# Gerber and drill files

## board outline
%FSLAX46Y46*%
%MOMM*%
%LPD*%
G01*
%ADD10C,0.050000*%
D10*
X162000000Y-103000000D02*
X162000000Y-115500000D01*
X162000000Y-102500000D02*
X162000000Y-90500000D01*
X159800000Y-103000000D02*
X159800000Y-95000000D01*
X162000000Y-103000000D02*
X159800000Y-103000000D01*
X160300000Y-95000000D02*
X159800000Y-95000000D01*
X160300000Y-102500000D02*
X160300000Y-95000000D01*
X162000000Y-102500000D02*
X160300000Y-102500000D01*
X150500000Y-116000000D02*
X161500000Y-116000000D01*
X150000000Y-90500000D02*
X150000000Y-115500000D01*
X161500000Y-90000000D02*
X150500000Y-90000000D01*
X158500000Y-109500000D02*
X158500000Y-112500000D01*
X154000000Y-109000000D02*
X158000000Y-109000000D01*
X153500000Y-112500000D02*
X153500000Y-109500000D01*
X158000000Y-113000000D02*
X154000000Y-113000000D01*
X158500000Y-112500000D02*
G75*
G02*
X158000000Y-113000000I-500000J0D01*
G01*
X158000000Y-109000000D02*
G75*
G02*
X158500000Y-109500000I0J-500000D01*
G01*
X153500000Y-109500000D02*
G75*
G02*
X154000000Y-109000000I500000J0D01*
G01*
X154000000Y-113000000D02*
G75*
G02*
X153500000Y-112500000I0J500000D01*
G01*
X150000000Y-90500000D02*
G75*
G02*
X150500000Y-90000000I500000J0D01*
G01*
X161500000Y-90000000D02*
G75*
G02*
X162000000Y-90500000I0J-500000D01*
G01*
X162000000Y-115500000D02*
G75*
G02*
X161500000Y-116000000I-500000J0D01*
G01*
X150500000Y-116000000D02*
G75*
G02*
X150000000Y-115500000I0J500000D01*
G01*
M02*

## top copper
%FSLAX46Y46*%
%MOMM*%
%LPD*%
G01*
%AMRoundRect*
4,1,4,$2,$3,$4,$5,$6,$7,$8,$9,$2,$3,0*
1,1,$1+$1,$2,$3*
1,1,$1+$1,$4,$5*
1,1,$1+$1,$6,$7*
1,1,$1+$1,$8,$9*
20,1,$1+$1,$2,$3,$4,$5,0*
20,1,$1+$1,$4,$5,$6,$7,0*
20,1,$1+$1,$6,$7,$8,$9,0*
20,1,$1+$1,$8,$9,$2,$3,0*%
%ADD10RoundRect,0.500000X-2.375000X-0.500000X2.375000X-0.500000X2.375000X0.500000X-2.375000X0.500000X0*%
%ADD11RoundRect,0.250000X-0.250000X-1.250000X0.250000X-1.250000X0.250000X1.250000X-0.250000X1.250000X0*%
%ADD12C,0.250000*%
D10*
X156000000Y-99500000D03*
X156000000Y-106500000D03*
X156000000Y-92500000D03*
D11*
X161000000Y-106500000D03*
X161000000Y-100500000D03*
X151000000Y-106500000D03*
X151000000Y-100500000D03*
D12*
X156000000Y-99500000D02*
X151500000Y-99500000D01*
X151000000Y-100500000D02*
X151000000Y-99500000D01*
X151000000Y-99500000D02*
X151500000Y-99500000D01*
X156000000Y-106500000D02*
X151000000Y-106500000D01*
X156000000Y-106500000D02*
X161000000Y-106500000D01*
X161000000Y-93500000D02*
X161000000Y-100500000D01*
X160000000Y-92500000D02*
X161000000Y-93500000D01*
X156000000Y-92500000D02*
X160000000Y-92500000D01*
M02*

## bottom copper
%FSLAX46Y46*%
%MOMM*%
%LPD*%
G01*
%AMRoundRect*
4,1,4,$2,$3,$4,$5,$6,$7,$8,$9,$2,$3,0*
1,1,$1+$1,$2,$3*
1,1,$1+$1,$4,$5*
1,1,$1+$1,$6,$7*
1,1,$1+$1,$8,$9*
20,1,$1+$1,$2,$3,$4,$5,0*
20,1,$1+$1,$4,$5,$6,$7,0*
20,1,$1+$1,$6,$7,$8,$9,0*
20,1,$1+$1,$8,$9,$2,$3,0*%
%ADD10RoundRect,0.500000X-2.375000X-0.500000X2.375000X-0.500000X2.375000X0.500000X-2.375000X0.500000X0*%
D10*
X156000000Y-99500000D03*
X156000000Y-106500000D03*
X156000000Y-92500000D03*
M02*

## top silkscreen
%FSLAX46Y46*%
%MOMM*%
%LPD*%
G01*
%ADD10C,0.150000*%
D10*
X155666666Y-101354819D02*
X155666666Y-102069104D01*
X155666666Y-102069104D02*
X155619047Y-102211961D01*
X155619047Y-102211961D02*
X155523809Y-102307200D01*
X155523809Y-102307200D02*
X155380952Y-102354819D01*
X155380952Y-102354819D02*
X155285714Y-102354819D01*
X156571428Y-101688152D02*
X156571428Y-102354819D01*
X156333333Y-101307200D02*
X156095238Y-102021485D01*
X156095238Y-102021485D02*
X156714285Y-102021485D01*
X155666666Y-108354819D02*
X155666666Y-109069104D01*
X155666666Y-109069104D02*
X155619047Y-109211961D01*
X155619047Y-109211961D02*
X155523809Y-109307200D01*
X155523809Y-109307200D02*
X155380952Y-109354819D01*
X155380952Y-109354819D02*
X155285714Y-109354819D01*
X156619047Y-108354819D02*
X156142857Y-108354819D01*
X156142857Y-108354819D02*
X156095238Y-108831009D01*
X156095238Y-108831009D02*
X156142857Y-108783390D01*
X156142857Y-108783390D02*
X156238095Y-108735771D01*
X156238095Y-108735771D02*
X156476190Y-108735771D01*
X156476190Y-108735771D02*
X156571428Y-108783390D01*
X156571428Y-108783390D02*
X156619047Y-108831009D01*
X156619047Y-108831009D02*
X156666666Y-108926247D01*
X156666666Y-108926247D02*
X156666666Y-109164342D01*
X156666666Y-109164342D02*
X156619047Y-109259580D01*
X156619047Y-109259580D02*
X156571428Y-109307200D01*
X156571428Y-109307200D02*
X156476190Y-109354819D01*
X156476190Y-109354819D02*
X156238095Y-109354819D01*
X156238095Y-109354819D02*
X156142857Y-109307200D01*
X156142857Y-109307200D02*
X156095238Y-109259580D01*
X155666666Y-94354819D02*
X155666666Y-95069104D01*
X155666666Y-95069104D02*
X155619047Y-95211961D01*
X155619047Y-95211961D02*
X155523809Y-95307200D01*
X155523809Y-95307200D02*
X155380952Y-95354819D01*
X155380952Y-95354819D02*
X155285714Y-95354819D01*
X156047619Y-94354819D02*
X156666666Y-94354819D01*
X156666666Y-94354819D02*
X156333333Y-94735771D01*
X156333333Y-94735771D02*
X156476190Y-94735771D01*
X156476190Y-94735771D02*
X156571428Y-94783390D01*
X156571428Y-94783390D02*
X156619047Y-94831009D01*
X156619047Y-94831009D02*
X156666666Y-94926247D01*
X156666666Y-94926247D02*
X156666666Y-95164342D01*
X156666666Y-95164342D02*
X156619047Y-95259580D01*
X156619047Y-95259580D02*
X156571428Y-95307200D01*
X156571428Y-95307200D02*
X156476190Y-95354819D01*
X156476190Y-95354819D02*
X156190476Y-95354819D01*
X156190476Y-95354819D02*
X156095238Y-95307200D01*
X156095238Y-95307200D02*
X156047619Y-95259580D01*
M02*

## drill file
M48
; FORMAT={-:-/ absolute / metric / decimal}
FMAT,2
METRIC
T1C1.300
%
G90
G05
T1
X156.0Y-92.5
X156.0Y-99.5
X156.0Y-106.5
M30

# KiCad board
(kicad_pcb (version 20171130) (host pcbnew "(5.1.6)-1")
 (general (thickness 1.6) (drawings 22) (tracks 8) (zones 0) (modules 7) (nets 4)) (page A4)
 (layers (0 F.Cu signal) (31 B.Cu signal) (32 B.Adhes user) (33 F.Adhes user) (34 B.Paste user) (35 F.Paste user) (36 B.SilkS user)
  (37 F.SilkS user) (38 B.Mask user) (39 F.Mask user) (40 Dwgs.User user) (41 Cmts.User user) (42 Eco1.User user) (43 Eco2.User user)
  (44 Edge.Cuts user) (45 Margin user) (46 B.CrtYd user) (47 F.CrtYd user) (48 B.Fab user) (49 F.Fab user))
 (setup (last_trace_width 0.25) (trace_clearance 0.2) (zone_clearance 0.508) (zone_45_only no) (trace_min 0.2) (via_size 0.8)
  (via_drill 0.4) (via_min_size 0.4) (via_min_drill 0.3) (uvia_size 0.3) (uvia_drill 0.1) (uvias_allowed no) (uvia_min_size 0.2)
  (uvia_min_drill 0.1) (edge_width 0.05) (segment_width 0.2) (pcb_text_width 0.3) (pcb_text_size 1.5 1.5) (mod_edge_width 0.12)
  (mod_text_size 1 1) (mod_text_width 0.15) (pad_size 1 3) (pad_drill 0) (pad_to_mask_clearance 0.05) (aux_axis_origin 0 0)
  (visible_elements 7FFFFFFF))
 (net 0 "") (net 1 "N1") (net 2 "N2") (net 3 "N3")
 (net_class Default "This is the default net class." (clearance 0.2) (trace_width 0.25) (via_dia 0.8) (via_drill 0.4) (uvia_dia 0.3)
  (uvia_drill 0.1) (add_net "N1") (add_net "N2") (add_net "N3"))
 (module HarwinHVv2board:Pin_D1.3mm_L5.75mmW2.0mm (layer F.Cu) (at 156 99.5)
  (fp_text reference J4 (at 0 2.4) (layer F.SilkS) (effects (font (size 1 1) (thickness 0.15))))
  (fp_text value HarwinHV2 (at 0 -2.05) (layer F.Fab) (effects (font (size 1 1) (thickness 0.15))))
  (pad 1 thru_hole roundrect (at 0 0) (size 5.75 2) (drill 1.3) (layers *.Cu *.Mask) (roundrect_rratio 0.25) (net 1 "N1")))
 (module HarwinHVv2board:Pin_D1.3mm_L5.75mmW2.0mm (layer F.Cu) (at 156 106.5)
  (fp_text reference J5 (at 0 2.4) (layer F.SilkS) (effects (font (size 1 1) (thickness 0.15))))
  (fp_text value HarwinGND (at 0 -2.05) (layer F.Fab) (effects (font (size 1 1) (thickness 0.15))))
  (pad 1 thru_hole roundrect (at 0 0) (size 5.75 2) (drill 1.3) (layers *.Cu *.Mask) (roundrect_rratio 0.25) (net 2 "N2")))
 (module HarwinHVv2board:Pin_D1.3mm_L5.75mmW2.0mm (layer F.Cu) (at 156 92.5)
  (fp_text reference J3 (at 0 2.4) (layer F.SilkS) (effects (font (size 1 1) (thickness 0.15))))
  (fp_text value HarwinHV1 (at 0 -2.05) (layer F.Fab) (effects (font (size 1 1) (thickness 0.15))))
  (pad 1 thru_hole roundrect (at 0 0) (size 5.75 2) (drill 1.3) (layers *.Cu *.Mask) (roundrect_rratio 0.25) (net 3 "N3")))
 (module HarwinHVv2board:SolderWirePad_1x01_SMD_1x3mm (layer F.Cu) (at 161 106.5)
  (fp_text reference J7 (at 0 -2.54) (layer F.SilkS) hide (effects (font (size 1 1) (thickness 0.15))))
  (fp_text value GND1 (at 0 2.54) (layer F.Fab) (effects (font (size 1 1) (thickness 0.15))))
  (pad 1 smd roundrect (at 0 0) (size 1 3) (layers F.Cu F.Paste F.Mask) (roundrect_rratio 0.25) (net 2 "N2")))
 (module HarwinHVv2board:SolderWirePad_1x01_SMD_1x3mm (layer F.Cu) (at 161 100.5)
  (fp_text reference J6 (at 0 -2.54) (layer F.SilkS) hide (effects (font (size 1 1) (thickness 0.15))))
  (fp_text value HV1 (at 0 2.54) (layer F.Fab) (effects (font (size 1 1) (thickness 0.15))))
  (pad 1 smd roundrect (at 0 0) (size 1 3) (layers F.Cu F.Paste F.Mask) (roundrect_rratio 0.25) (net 3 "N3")))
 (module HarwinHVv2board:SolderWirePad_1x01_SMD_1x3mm (layer F.Cu) (at 151 106.5)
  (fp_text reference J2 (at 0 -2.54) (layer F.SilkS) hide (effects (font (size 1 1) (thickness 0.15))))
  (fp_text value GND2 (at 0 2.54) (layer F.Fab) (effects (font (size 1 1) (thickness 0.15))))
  (pad 1 smd roundrect (at 0 0) (size 1 3) (layers F.Cu F.Paste F.Mask) (roundrect_rratio 0.25) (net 2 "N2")))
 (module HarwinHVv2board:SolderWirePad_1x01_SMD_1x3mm (layer F.Cu) (at 151 100.5)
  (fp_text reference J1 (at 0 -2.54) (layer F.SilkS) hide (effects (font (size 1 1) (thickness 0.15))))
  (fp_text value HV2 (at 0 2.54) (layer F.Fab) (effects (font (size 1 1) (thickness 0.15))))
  (pad 1 smd roundrect (at 0 0) (size 1 3) (layers F.Cu F.Paste F.Mask) (roundrect_rratio 0.25) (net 1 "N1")))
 (gr_line (start 162 103) (end 162 115.5) (layer Edge.Cuts) (width 0.05))
 (gr_line (start 162 102.5) (end 162 90.5) (layer Edge.Cuts) (width 0.05))
 (gr_line (start 159.8 103) (end 159.8 95) (layer Edge.Cuts) (width 0.05))
 (gr_line (start 162 103) (end 159.8 103) (layer Edge.Cuts) (width 0.05))
 (gr_line (start 160.3 95) (end 159.8 95) (layer Edge.Cuts) (width 0.05))
 (gr_line (start 160.3 102.5) (end 160.3 95) (layer Edge.Cuts) (width 0.05))
 (gr_line (start 162 102.5) (end 160.3 102.5) (layer Edge.Cuts) (width 0.05))
 (gr_line (start 150.5 116) (end 161.5 116) (layer Edge.Cuts) (width 0.05))
 (gr_line (start 150 90.5) (end 150 115.5) (layer Edge.Cuts) (width 0.05))
 (gr_line (start 161.5 90) (end 150.5 90) (layer Edge.Cuts) (width 0.05))
 (gr_line (start 158.5 109.5) (end 158.5 112.5) (layer Edge.Cuts) (width 0.05))
 (gr_line (start 154 109) (end 158 109) (layer Edge.Cuts) (width 0.05))
 (gr_line (start 153.5 112.5) (end 153.5 109.5) (layer Edge.Cuts) (width 0.05))
 (gr_line (start 158 113) (end 154 113) (layer Edge.Cuts) (width 0.05))
 (gr_arc (start 158 112.5) (end 158.5 112.5) (angle 90) (layer Edge.Cuts) (width 0.05))
 (gr_arc (start 158 109.5) (end 158 109) (angle 90) (layer Edge.Cuts) (width 0.05))
 (gr_arc (start 154 109.5) (end 153.5 109.5) (angle 90) (layer Edge.Cuts) (width 0.05))
 (gr_arc (start 154 112.5) (end 154 113) (angle 90) (layer Edge.Cuts) (width 0.05))
 (gr_arc (start 150.5 90.5) (end 150 90.5) (angle 90) (layer Edge.Cuts) (width 0.05))
 (gr_arc (start 161.5 90.5) (end 161.5 90) (angle 90) (layer Edge.Cuts) (width 0.05))
 (gr_arc (start 161.5 115.5) (end 162 115.5) (angle 90) (layer Edge.Cuts) (width 0.05))
 (gr_arc (start 150.5 115.5) (end 150 115.5) (angle -90) (layer Edge.Cuts) (width 0.05))
 (segment (start 156 99.5) (end 151.5 99.5) (width 0.25) (layer F.Cu) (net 1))
 (segment (start 151 100.5) (end 151 99.5) (width 0.25) (layer F.Cu) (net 1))
 (segment (start 151 99.5) (end 151.5 99.5) (width 0.25) (layer F.Cu) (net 1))
 (segment (start 156 106.5) (end 151 106.5) (width 0.25) (layer F.Cu) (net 2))
 (segment (start 156 106.5) (end 161 106.5) (width 0.25) (layer F.Cu) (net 2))
 (segment (start 161 93.5) (end 161 100.5) (width 0.25) (layer F.Cu) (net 3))
 (segment (start 160 92.5) (end 161 93.5) (width 0.25) (layer F.Cu) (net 3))
 (segment (start 156 92.5) (end 160 92.5) (width 0.25) (layer F.Cu) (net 3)))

